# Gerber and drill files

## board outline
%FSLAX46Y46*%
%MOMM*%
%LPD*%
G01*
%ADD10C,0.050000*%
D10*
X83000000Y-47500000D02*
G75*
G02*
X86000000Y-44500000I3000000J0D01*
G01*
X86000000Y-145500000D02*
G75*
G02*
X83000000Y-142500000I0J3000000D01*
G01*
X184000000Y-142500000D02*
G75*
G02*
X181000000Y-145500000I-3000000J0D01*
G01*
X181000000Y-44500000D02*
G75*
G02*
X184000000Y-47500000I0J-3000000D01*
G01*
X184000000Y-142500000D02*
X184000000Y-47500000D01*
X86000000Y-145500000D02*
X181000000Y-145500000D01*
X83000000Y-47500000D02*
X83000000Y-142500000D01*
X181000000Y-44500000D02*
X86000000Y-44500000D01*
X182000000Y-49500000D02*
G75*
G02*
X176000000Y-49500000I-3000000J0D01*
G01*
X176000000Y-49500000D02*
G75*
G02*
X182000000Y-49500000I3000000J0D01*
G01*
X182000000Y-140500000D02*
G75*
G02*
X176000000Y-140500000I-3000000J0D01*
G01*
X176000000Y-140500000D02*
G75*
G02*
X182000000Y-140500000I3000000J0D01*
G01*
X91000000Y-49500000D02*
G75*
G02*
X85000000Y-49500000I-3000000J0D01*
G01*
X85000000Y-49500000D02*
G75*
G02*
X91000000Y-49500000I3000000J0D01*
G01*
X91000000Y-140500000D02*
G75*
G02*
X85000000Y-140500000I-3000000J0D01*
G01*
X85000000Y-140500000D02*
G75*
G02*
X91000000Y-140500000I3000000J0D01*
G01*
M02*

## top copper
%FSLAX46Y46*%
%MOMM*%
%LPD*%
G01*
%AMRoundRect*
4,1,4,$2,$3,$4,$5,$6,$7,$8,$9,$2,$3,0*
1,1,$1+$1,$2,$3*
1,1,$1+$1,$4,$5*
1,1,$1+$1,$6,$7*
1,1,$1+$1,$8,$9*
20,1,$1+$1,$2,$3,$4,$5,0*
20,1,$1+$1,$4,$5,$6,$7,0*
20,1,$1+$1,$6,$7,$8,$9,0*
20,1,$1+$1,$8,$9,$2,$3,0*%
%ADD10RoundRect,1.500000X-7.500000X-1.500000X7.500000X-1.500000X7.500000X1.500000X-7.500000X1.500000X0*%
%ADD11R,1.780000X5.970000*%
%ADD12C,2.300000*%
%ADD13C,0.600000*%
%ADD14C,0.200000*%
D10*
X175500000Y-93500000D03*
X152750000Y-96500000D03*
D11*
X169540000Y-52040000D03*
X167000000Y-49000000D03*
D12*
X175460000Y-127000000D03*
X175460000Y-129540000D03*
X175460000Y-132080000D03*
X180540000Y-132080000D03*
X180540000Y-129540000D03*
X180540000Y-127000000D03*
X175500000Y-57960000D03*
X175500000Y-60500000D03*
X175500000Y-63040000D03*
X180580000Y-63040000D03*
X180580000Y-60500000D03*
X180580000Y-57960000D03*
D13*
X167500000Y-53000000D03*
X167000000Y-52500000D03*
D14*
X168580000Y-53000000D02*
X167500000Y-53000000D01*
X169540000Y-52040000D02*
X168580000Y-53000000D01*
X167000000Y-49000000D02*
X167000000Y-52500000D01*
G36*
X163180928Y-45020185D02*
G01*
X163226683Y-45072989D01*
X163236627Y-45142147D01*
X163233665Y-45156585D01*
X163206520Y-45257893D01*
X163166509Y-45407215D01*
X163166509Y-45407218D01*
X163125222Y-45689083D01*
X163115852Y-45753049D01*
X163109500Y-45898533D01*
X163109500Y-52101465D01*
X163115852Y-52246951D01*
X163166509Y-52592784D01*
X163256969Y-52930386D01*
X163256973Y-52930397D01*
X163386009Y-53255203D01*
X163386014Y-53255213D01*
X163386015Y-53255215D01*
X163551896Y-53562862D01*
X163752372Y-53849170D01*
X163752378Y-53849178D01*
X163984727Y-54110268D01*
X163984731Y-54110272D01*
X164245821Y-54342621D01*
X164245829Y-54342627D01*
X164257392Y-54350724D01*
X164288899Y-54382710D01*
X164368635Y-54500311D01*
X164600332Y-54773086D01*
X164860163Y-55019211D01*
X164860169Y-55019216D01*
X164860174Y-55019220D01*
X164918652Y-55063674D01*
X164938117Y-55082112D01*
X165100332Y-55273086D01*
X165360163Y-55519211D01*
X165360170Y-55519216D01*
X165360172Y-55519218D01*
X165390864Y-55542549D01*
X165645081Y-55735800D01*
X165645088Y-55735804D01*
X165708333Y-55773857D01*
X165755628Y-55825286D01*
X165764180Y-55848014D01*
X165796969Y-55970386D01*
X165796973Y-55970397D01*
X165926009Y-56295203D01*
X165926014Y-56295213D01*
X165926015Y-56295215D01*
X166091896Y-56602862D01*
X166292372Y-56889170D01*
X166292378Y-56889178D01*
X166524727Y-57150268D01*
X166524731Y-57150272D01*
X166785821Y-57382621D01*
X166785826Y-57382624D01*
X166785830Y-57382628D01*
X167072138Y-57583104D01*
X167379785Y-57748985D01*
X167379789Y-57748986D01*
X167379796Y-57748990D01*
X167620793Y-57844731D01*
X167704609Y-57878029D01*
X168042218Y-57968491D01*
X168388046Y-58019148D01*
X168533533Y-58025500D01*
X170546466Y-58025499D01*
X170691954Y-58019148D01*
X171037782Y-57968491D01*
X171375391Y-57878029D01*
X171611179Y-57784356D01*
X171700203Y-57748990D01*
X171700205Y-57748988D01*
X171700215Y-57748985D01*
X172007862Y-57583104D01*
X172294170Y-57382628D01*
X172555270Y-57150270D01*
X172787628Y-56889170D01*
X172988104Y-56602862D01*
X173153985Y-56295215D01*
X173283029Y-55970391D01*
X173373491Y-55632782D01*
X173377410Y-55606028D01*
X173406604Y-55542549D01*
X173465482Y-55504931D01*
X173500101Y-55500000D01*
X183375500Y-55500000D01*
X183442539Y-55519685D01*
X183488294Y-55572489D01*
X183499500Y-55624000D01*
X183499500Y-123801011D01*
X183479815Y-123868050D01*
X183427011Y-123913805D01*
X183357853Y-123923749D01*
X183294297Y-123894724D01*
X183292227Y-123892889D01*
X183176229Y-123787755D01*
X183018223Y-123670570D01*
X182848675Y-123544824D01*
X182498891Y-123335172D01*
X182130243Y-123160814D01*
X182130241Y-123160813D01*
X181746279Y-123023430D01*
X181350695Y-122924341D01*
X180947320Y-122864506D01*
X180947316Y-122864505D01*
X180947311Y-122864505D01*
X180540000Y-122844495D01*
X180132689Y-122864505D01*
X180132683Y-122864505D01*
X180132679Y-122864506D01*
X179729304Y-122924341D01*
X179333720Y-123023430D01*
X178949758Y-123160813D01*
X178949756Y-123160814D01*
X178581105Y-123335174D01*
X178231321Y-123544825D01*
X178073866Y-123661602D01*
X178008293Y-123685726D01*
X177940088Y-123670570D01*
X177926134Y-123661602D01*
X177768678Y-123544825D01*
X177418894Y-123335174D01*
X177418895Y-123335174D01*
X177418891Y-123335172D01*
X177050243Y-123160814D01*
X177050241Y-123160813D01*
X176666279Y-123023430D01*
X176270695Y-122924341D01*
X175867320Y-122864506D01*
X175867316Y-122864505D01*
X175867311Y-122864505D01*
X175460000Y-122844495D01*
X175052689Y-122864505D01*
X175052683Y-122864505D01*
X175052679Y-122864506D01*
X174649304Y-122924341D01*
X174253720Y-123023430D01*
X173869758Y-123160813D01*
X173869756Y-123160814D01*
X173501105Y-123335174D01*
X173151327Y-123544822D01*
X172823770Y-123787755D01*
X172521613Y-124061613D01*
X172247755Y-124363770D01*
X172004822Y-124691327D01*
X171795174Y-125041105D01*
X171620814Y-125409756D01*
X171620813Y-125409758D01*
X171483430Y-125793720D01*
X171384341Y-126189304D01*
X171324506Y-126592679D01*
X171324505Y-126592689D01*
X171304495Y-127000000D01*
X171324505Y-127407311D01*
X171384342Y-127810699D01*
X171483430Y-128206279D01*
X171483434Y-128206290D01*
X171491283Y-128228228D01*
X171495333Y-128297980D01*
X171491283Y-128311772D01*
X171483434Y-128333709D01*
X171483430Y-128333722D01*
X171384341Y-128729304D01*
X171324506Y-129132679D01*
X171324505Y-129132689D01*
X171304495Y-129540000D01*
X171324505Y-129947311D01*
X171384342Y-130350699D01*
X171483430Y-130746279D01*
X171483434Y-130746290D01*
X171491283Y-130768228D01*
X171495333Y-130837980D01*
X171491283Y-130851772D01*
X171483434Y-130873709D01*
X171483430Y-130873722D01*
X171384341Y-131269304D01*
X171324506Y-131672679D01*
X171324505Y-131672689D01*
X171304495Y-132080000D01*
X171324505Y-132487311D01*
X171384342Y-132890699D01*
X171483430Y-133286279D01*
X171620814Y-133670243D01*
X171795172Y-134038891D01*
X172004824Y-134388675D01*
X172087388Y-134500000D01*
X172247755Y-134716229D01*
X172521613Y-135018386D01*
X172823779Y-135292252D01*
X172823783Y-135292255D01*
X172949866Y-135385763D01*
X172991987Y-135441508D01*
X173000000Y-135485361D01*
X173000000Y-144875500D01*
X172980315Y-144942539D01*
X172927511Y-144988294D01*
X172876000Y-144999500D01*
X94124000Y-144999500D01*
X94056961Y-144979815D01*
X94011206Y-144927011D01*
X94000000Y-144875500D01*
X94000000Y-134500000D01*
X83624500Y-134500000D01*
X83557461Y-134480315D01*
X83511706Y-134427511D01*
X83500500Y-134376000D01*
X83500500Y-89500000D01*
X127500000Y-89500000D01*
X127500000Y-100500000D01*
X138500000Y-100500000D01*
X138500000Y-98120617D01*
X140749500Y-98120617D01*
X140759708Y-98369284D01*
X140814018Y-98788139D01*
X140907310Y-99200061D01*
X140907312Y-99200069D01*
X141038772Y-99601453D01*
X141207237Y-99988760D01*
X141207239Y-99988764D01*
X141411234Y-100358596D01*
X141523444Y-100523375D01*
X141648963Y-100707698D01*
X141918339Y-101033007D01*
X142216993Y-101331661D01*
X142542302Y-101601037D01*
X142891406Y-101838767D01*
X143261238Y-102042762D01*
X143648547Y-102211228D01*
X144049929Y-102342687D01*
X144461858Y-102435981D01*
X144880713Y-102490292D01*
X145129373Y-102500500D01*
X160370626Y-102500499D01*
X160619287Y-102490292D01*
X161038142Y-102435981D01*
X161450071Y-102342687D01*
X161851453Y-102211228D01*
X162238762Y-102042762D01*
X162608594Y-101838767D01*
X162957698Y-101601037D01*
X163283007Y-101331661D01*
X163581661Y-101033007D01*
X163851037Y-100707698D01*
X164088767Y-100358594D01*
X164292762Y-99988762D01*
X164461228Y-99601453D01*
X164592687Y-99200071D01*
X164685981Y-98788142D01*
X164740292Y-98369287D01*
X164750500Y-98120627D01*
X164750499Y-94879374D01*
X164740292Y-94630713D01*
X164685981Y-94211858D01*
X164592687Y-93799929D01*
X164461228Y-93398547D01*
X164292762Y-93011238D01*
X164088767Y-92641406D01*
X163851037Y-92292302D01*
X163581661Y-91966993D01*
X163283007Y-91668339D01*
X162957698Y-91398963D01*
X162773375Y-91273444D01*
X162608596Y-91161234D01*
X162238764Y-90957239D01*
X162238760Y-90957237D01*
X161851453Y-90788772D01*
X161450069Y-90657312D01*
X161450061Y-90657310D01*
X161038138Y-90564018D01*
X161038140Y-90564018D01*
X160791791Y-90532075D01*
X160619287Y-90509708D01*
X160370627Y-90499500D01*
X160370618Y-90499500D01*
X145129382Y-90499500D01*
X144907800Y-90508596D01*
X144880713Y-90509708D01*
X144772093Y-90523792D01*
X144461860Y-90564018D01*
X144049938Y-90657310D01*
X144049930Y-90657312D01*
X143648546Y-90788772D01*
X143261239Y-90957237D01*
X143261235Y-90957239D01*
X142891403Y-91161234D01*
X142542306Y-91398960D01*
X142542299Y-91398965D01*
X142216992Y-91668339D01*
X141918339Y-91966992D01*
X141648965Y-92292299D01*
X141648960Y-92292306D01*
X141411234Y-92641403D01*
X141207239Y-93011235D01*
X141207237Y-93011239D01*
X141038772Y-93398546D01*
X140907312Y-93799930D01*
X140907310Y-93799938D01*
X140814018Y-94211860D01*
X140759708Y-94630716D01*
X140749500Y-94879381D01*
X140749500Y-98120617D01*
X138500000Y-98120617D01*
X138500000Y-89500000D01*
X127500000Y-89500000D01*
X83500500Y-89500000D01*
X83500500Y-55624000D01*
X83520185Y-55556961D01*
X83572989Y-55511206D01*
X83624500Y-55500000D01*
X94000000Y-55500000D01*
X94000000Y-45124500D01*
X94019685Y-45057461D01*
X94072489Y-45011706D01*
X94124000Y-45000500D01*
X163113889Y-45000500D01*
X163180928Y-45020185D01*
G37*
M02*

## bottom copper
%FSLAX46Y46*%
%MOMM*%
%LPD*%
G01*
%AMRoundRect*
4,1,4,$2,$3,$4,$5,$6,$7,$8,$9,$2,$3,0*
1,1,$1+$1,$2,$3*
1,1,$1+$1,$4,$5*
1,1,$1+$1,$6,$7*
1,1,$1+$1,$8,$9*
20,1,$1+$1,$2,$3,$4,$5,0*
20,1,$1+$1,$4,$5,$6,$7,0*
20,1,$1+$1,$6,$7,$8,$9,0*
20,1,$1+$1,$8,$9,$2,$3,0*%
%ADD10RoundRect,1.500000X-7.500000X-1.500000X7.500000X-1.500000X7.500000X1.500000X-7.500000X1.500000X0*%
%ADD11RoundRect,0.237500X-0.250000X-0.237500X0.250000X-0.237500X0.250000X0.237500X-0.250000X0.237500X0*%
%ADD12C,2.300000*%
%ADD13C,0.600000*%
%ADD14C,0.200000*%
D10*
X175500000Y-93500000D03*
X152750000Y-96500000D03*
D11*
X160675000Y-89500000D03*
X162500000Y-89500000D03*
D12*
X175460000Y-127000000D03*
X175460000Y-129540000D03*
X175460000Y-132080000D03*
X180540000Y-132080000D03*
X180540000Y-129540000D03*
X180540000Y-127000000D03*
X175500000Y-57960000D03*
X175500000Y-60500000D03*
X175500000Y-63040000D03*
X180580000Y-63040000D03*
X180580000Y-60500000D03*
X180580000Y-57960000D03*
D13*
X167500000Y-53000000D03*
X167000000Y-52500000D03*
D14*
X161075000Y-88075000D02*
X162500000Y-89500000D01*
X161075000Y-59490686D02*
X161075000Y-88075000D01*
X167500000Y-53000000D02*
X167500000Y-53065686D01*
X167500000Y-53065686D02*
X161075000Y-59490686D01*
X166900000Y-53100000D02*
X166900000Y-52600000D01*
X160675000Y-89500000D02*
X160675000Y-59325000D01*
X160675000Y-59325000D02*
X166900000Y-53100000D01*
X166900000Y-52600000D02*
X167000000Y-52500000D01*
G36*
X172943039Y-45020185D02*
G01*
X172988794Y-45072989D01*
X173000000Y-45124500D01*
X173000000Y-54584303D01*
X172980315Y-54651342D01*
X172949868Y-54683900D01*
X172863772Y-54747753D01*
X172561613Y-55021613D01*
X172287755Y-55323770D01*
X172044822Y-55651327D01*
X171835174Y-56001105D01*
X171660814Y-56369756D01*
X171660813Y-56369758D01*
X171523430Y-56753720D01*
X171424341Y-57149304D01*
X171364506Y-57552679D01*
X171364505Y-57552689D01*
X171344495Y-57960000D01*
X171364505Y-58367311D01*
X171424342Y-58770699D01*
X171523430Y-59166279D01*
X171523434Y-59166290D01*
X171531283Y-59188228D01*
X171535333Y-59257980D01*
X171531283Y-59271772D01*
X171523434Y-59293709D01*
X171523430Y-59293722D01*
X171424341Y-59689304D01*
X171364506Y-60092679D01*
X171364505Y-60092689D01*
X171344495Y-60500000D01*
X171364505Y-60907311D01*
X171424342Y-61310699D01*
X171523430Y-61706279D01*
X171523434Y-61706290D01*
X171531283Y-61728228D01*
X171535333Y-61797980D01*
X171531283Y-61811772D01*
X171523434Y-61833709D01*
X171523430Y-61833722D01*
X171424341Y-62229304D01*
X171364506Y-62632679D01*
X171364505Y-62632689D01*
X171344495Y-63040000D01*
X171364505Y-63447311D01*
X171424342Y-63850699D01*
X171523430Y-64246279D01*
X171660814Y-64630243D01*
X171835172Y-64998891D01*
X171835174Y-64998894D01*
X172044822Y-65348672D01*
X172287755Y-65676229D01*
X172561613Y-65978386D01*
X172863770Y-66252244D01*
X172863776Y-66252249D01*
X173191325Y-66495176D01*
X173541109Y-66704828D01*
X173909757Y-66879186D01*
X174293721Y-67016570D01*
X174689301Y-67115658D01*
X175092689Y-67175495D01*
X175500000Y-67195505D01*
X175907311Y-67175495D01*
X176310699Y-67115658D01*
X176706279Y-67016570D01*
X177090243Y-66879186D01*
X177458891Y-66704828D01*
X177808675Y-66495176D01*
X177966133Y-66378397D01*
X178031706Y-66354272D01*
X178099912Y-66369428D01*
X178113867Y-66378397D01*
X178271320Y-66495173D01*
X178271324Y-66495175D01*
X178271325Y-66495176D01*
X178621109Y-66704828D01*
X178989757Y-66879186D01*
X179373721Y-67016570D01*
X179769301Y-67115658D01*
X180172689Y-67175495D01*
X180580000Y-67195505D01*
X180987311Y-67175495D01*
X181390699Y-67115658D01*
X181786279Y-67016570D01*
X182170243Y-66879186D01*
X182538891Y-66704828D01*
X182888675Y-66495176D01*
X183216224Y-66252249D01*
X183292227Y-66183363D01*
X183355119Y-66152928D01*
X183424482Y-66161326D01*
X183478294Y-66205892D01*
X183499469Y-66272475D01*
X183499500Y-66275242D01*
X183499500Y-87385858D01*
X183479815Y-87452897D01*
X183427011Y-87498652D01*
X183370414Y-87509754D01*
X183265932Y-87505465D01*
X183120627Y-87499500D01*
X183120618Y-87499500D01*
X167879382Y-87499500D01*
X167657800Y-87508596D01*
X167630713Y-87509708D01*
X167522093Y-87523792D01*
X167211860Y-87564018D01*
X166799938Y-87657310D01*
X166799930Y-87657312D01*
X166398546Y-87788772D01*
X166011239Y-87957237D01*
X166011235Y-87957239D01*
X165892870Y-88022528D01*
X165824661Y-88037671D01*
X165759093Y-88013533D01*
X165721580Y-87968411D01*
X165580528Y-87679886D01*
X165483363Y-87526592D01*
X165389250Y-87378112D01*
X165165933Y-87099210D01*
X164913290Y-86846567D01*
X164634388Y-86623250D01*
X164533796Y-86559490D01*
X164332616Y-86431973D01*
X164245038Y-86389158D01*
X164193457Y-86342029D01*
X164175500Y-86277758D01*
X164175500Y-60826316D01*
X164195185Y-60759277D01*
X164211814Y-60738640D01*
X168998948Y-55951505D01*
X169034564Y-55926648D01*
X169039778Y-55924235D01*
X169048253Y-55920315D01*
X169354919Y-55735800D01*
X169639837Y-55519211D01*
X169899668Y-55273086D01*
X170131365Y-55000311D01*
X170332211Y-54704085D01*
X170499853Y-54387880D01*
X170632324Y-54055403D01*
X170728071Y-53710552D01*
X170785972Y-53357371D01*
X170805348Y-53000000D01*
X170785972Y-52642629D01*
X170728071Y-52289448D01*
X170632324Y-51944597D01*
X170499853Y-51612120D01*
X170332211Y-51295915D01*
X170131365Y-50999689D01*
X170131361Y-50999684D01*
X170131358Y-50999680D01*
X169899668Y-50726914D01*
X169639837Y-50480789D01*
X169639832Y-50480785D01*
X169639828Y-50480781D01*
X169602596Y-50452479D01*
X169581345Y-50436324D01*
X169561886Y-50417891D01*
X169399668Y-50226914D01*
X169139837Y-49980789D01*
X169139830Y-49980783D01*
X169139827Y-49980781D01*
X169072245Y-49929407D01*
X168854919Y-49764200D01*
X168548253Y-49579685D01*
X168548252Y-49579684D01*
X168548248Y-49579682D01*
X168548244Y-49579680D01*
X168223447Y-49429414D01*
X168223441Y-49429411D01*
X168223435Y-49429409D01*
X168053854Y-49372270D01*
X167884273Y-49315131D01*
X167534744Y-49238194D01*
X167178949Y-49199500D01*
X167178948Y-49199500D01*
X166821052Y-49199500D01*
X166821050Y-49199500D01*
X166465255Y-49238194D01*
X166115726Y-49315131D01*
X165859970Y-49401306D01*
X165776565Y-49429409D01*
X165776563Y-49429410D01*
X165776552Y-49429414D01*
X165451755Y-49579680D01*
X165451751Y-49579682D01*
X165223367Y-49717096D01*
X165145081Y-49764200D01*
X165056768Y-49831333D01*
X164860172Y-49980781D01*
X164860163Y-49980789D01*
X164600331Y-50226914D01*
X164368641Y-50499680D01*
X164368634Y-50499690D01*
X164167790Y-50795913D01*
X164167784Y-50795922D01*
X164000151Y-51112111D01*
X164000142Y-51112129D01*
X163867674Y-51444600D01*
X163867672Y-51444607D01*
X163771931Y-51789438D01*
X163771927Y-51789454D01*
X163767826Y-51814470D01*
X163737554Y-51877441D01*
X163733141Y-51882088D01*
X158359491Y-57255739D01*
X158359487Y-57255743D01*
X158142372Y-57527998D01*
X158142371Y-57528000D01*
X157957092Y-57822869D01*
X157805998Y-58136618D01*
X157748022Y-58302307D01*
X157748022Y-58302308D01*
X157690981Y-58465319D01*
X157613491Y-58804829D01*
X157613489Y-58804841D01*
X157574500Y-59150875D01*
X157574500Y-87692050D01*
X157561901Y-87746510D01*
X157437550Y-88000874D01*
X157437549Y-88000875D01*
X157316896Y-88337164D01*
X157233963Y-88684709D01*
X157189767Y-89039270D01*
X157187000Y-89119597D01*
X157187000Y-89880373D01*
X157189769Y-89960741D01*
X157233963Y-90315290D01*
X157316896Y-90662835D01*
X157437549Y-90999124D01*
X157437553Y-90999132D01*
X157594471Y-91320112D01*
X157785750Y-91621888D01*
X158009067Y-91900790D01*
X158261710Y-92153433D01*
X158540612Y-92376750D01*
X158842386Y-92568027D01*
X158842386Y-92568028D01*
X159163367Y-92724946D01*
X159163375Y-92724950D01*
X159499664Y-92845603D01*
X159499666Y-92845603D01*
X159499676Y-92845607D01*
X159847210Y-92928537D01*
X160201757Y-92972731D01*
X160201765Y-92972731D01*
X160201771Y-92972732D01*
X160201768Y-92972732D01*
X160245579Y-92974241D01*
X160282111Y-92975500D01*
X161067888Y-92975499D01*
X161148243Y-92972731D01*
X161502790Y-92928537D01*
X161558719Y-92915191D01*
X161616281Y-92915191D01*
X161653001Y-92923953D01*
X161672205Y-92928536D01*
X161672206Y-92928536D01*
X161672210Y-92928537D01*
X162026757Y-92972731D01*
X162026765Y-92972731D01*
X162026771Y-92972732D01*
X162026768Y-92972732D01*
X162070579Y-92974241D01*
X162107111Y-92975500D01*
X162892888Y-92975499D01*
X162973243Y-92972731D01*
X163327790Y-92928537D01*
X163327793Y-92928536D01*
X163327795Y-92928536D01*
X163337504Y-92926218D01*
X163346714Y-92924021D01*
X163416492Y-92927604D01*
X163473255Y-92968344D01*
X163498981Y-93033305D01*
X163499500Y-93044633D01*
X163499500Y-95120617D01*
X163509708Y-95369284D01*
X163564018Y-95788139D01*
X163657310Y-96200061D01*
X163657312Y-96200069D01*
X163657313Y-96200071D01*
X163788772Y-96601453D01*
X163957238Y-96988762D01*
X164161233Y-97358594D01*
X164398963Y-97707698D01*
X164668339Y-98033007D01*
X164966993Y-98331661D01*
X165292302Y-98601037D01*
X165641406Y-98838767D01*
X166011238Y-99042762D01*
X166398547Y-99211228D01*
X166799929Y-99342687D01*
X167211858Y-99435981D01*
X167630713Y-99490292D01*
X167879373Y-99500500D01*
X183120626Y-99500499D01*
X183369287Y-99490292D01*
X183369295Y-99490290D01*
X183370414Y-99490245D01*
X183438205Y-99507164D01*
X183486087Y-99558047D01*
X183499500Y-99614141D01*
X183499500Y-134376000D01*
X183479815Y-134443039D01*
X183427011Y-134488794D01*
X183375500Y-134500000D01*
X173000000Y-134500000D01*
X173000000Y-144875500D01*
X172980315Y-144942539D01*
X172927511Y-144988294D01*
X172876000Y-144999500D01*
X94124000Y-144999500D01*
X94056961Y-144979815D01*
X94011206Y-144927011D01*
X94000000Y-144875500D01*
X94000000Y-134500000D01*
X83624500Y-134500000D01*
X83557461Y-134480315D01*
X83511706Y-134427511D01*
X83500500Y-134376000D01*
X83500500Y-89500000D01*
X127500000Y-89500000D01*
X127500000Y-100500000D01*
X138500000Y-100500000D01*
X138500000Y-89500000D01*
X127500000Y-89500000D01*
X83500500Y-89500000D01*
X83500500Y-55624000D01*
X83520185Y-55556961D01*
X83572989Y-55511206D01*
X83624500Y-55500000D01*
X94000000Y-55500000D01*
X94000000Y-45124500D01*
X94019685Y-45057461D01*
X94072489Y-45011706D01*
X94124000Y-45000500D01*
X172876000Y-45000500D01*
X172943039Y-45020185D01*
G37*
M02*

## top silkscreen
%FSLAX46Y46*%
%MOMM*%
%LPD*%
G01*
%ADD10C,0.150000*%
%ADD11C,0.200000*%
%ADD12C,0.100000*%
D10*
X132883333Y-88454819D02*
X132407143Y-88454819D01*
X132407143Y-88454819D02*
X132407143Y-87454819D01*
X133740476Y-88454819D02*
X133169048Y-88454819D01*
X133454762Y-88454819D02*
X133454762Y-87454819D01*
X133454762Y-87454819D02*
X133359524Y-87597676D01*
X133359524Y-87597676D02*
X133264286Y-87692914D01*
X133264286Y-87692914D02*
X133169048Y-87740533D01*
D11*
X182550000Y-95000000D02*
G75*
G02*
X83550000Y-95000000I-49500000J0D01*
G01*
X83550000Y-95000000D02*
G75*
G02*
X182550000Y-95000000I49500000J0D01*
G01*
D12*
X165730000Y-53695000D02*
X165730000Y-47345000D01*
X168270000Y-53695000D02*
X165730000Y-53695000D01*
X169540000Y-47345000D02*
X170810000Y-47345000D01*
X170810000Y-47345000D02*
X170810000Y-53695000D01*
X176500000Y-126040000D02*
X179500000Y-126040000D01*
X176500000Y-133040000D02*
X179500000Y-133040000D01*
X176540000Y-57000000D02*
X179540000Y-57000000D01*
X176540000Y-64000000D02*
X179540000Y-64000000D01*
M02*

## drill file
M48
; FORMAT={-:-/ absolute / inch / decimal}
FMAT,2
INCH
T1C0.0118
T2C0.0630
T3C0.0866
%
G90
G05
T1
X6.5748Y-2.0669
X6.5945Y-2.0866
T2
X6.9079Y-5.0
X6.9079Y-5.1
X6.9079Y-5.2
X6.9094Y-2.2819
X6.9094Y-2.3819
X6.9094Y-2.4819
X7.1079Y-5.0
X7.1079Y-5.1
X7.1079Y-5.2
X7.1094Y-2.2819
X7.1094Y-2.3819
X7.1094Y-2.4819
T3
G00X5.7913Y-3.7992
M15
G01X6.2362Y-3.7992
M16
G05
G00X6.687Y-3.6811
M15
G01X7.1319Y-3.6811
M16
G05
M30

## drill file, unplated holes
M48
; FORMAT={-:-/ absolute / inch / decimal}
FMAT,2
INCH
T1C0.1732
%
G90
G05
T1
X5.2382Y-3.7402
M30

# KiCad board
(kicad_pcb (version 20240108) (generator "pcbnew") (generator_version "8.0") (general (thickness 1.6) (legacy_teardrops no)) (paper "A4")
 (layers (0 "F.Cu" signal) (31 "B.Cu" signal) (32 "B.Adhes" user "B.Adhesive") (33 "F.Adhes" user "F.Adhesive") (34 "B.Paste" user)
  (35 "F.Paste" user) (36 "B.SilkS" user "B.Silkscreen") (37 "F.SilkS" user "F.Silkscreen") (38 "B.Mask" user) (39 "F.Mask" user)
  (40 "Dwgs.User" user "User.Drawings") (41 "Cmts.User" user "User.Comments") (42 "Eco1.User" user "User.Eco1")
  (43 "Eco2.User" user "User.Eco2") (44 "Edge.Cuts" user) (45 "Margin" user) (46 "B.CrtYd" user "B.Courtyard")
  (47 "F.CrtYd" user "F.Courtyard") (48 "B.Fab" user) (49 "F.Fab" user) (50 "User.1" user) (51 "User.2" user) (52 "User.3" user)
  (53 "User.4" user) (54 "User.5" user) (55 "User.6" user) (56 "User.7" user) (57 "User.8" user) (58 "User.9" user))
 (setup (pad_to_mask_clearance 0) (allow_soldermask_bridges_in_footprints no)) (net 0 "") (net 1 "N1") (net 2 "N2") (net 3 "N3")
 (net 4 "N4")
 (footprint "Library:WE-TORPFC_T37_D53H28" (layer "F.Cu") (at 133.05 95)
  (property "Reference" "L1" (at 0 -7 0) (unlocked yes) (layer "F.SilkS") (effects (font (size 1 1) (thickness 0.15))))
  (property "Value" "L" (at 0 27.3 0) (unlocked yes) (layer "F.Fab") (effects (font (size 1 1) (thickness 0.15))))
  (fp_circle (center 0 0) (end 49.5 0) (stroke (width 0.2) (type solid)) (fill none) (layer "F.SilkS"))
  (pad "" np_thru_hole circle (at 0 0) (size 4.4 4.4) (drill 4.4) (layers "F&B.Cu" "*.Mask"))
  (pad "1" thru_hole roundrect (at 42.45 -1.5) (size 18 6) (drill oval 13.5 2.2) (layers "*.Cu" "*.Mask") (remove_unused_layers no)
   (roundrect_rratio 0.25) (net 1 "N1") (thermal_bridge_angle 45))
  (pad "2" thru_hole roundrect (at 19.7 1.5) (size 18 6) (drill oval 13.5 2.2) (layers "*.Cu" "*.Mask") (remove_unused_layers no)
   (roundrect_rratio 0.25) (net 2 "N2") (thermal_bridge_angle 45)))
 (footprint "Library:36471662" (layer "F.Cu") (at 168.27 50.52)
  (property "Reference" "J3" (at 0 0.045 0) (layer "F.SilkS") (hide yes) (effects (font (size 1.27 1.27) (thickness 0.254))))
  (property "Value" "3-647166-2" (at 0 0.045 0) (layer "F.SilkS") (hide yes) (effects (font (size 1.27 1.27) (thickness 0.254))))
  (fp_line (start -2.54 3.175) (end -2.54 -3.175) (stroke (width 0.1) (type solid)) (layer "F.SilkS"))
  (fp_line (start 0 3.175) (end -2.54 3.175) (stroke (width 0.1) (type solid)) (layer "F.SilkS"))
  (fp_line (start 1.27 -3.175) (end 2.54 -3.175) (stroke (width 0.1) (type solid)) (layer "F.SilkS"))
  (fp_line (start 2.54 -3.175) (end 2.54 3.175) (stroke (width 0.1) (type solid)) (layer "F.SilkS"))
  (pad "1" smd rect (at 1.27 1.52) (size 1.78 5.97) (layers "F.Cu" "F.Paste" "F.Mask") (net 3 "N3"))
  (pad "2" smd rect (at -1.27 -1.52) (size 1.78 5.97) (layers "F.Cu" "F.Paste" "F.Mask") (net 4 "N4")))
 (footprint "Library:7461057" (layer "F.Cu") (at 175.46 127)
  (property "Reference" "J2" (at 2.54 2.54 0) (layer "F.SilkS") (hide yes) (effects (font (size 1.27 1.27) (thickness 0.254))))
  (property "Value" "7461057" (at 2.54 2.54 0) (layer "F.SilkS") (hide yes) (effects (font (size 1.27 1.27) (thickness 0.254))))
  (fp_line (start 1.04 -0.96) (end 4.04 -0.96) (stroke (width 0.1) (type solid)) (layer "F.SilkS"))
  (fp_line (start 1.04 6.04) (end 4.04 6.04) (stroke (width 0.1) (type solid)) (layer "F.SilkS"))
  (pad "1" thru_hole circle (at 0 0) (size 2.3 2.3) (drill 1.6) (layers "*.Cu" "*.Mask") (remove_unused_layers no) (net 2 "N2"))
  (pad "2" thru_hole circle (at 0 2.54) (size 2.3 2.3) (drill 1.6) (layers "*.Cu" "*.Mask") (remove_unused_layers no) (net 2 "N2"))
  (pad "3" thru_hole circle (at 0 5.08) (size 2.3 2.3) (drill 1.6) (layers "*.Cu" "*.Mask") (remove_unused_layers no) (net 2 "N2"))
  (pad "4" thru_hole circle (at 5.08 5.08) (size 2.3 2.3) (drill 1.6) (layers "*.Cu" "*.Mask") (remove_unused_layers no) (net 2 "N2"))
  (pad "5" thru_hole circle (at 5.08 2.54) (size 2.3 2.3) (drill 1.6) (layers "*.Cu" "*.Mask") (remove_unused_layers no) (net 2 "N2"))
  (pad "6" thru_hole circle (at 5.08 0) (size 2.3 2.3) (drill 1.6) (layers "*.Cu" "*.Mask") (remove_unused_layers no) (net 2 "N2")))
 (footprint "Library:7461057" (layer "F.Cu") (at 175.5 57.96)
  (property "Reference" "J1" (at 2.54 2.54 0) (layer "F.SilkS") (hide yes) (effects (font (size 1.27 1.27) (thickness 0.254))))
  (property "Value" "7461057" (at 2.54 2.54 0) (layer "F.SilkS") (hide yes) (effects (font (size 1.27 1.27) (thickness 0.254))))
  (fp_line (start 1.04 -0.96) (end 4.04 -0.96) (stroke (width 0.1) (type solid)) (layer "F.SilkS"))
  (fp_line (start 1.04 6.04) (end 4.04 6.04) (stroke (width 0.1) (type solid)) (layer "F.SilkS"))
  (pad "1" thru_hole circle (at 0 0) (size 2.3 2.3) (drill 1.6) (layers "*.Cu" "*.Mask") (remove_unused_layers no) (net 1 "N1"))
  (pad "2" thru_hole circle (at 0 2.54) (size 2.3 2.3) (drill 1.6) (layers "*.Cu" "*.Mask") (remove_unused_layers no) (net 1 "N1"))
  (pad "3" thru_hole circle (at 0 5.08) (size 2.3 2.3) (drill 1.6) (layers "*.Cu" "*.Mask") (remove_unused_layers no) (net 1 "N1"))
  (pad "4" thru_hole circle (at 5.08 5.08) (size 2.3 2.3) (drill 1.6) (layers "*.Cu" "*.Mask") (remove_unused_layers no) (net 1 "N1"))
  (pad "5" thru_hole circle (at 5.08 2.54) (size 2.3 2.3) (drill 1.6) (layers "*.Cu" "*.Mask") (remove_unused_layers no) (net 1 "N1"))
  (pad "6" thru_hole circle (at 5.08 0) (size 2.3 2.3) (drill 1.6) (layers "*.Cu" "*.Mask") (remove_unused_layers no) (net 1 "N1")))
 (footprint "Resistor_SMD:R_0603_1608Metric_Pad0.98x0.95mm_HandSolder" (layer "B.Cu") (at 161.5875 89.5)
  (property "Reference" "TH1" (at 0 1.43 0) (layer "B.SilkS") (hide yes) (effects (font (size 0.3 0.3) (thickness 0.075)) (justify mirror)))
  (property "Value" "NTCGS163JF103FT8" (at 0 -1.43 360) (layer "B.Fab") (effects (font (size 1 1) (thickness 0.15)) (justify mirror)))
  (pad "1" smd roundrect (at -0.9125 0) (size 0.975 0.95) (layers "B.Cu" "B.Paste" "B.Mask") (roundrect_rratio 0.25) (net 4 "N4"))
  (pad "2" smd roundrect (at 0.9125 0) (size 0.975 0.95) (layers "B.Cu" "B.Paste" "B.Mask") (roundrect_rratio 0.25) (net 3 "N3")))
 (gr_circle (center 179 49.5) (end 182 49.5) (stroke (width 0.05) (type default)) (fill none) (layer "Edge.Cuts"))
 (gr_line (start 86 145.5) (end 181 145.5) (stroke (width 0.05) (type default)) (layer "Edge.Cuts"))
 (gr_arc (start 83 47.5) (mid 83.87868 45.37868) (end 86 44.5) (stroke (width 0.05) (type default)) (layer "Edge.Cuts"))
 (gr_circle (center 179 140.5) (end 182 140.5) (stroke (width 0.05) (type default)) (fill none) (layer "Edge.Cuts"))
 (gr_arc (start 184 142.5) (mid 183.12132 144.62132) (end 181 145.5) (stroke (width 0.05) (type default)) (layer "Edge.Cuts"))
 (gr_circle (center 88 49.5) (end 91 49.5) (stroke (width 0.05) (type default)) (fill none) (layer "Edge.Cuts"))
 (gr_circle (center 88 140.5) (end 91 140.5) (stroke (width 0.05) (type default)) (fill none) (layer "Edge.Cuts"))
 (gr_arc (start 86 145.5) (mid 83.87868 144.62132) (end 83 142.5) (stroke (width 0.05) (type default)) (layer "Edge.Cuts"))
 (gr_line (start 181 44.5) (end 86 44.5) (stroke (width 0.05) (type default)) (layer "Edge.Cuts"))
 (gr_line (start 184 142.5) (end 184 47.5) (stroke (width 0.05) (type default)) (layer "Edge.Cuts"))
 (gr_line (start 83 47.5) (end 83 142.5) (stroke (width 0.05) (type default)) (layer "Edge.Cuts"))
 (gr_arc (start 181 44.5) (mid 183.12132 45.37868) (end 184 47.5) (stroke (width 0.05) (type default)) (layer "Edge.Cuts"))
 (segment (start 167 49) (end 167 52.5) (width 0.2) (layer "F.Cu") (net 4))
 (via (at 167 52.5) (size 0.6) (drill 0.3) (layers "F.Cu" "B.Cu") (free yes) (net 4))
 (segment (start 166.9 53.1) (end 166.9 52.6) (width 0.2) (layer "B.Cu") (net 4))
 (segment (start 166.9 52.6) (end 167 52.5) (width 0.2) (layer "B.Cu") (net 4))
 (segment (start 160.675 89.5) (end 160.675 59.325) (width 0.2) (layer "B.Cu") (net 4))
 (segment (start 160.675 59.325) (end 166.9 53.1) (width 0.2) (layer "B.Cu") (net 4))
 (segment (start 168.58 53) (end 167.5 53) (width 0.2) (layer "F.Cu") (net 3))
 (segment (start 169.54 52.04) (end 168.58 53) (width 0.2) (layer "F.Cu") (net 3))
 (via (at 167.5 53) (size 0.6) (drill 0.3) (layers "F.Cu" "B.Cu") (free yes) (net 3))
 (segment (start 161.075 59.490686) (end 161.075 88.075) (width 0.2) (layer "B.Cu") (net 3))
 (segment (start 167.5 53.065686) (end 161.075 59.490686) (width 0.2) (layer "B.Cu") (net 3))
 (segment (start 167.5 53) (end 167.5 53.065686) (width 0.2) (layer "B.Cu") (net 3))
 (segment (start 161.075 88.075) (end 162.5 89.5) (width 0.2) (layer "B.Cu") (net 3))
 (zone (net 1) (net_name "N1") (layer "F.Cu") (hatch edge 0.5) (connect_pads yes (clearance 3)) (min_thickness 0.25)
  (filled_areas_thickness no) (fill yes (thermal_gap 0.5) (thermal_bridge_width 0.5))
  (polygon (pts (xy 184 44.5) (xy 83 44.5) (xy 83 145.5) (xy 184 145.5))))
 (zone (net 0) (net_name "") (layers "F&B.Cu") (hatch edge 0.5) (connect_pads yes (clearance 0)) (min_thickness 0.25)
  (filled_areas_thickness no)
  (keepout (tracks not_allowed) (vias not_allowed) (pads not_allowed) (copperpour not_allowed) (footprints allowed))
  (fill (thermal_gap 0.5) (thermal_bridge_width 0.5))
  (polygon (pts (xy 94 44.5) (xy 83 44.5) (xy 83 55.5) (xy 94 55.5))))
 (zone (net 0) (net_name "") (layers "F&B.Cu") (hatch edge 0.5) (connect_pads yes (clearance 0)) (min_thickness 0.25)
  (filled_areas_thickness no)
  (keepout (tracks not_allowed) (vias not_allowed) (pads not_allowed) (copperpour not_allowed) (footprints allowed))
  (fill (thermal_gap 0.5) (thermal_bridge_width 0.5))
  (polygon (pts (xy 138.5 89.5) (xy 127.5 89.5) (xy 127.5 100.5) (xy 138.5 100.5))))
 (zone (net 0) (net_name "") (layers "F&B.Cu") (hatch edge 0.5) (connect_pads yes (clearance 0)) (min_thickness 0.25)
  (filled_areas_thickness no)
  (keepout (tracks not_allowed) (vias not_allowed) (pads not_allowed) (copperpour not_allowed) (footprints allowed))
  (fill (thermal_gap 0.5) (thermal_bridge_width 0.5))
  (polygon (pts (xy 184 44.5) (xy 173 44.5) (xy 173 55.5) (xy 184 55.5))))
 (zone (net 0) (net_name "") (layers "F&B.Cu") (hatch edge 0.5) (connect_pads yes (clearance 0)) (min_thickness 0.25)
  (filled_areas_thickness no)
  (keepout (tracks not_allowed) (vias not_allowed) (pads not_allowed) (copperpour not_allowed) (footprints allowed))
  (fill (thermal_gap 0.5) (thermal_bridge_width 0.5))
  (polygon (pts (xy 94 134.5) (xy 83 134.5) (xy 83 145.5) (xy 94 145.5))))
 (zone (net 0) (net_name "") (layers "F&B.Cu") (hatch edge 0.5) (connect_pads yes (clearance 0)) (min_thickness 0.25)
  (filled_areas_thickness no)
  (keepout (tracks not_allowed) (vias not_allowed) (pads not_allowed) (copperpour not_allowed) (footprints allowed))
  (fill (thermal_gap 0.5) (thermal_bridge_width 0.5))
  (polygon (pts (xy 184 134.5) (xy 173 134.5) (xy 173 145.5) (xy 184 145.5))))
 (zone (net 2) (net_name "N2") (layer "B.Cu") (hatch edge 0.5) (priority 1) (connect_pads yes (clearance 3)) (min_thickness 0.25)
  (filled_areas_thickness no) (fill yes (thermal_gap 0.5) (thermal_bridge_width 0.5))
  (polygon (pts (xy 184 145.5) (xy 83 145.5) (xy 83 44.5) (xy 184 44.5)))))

